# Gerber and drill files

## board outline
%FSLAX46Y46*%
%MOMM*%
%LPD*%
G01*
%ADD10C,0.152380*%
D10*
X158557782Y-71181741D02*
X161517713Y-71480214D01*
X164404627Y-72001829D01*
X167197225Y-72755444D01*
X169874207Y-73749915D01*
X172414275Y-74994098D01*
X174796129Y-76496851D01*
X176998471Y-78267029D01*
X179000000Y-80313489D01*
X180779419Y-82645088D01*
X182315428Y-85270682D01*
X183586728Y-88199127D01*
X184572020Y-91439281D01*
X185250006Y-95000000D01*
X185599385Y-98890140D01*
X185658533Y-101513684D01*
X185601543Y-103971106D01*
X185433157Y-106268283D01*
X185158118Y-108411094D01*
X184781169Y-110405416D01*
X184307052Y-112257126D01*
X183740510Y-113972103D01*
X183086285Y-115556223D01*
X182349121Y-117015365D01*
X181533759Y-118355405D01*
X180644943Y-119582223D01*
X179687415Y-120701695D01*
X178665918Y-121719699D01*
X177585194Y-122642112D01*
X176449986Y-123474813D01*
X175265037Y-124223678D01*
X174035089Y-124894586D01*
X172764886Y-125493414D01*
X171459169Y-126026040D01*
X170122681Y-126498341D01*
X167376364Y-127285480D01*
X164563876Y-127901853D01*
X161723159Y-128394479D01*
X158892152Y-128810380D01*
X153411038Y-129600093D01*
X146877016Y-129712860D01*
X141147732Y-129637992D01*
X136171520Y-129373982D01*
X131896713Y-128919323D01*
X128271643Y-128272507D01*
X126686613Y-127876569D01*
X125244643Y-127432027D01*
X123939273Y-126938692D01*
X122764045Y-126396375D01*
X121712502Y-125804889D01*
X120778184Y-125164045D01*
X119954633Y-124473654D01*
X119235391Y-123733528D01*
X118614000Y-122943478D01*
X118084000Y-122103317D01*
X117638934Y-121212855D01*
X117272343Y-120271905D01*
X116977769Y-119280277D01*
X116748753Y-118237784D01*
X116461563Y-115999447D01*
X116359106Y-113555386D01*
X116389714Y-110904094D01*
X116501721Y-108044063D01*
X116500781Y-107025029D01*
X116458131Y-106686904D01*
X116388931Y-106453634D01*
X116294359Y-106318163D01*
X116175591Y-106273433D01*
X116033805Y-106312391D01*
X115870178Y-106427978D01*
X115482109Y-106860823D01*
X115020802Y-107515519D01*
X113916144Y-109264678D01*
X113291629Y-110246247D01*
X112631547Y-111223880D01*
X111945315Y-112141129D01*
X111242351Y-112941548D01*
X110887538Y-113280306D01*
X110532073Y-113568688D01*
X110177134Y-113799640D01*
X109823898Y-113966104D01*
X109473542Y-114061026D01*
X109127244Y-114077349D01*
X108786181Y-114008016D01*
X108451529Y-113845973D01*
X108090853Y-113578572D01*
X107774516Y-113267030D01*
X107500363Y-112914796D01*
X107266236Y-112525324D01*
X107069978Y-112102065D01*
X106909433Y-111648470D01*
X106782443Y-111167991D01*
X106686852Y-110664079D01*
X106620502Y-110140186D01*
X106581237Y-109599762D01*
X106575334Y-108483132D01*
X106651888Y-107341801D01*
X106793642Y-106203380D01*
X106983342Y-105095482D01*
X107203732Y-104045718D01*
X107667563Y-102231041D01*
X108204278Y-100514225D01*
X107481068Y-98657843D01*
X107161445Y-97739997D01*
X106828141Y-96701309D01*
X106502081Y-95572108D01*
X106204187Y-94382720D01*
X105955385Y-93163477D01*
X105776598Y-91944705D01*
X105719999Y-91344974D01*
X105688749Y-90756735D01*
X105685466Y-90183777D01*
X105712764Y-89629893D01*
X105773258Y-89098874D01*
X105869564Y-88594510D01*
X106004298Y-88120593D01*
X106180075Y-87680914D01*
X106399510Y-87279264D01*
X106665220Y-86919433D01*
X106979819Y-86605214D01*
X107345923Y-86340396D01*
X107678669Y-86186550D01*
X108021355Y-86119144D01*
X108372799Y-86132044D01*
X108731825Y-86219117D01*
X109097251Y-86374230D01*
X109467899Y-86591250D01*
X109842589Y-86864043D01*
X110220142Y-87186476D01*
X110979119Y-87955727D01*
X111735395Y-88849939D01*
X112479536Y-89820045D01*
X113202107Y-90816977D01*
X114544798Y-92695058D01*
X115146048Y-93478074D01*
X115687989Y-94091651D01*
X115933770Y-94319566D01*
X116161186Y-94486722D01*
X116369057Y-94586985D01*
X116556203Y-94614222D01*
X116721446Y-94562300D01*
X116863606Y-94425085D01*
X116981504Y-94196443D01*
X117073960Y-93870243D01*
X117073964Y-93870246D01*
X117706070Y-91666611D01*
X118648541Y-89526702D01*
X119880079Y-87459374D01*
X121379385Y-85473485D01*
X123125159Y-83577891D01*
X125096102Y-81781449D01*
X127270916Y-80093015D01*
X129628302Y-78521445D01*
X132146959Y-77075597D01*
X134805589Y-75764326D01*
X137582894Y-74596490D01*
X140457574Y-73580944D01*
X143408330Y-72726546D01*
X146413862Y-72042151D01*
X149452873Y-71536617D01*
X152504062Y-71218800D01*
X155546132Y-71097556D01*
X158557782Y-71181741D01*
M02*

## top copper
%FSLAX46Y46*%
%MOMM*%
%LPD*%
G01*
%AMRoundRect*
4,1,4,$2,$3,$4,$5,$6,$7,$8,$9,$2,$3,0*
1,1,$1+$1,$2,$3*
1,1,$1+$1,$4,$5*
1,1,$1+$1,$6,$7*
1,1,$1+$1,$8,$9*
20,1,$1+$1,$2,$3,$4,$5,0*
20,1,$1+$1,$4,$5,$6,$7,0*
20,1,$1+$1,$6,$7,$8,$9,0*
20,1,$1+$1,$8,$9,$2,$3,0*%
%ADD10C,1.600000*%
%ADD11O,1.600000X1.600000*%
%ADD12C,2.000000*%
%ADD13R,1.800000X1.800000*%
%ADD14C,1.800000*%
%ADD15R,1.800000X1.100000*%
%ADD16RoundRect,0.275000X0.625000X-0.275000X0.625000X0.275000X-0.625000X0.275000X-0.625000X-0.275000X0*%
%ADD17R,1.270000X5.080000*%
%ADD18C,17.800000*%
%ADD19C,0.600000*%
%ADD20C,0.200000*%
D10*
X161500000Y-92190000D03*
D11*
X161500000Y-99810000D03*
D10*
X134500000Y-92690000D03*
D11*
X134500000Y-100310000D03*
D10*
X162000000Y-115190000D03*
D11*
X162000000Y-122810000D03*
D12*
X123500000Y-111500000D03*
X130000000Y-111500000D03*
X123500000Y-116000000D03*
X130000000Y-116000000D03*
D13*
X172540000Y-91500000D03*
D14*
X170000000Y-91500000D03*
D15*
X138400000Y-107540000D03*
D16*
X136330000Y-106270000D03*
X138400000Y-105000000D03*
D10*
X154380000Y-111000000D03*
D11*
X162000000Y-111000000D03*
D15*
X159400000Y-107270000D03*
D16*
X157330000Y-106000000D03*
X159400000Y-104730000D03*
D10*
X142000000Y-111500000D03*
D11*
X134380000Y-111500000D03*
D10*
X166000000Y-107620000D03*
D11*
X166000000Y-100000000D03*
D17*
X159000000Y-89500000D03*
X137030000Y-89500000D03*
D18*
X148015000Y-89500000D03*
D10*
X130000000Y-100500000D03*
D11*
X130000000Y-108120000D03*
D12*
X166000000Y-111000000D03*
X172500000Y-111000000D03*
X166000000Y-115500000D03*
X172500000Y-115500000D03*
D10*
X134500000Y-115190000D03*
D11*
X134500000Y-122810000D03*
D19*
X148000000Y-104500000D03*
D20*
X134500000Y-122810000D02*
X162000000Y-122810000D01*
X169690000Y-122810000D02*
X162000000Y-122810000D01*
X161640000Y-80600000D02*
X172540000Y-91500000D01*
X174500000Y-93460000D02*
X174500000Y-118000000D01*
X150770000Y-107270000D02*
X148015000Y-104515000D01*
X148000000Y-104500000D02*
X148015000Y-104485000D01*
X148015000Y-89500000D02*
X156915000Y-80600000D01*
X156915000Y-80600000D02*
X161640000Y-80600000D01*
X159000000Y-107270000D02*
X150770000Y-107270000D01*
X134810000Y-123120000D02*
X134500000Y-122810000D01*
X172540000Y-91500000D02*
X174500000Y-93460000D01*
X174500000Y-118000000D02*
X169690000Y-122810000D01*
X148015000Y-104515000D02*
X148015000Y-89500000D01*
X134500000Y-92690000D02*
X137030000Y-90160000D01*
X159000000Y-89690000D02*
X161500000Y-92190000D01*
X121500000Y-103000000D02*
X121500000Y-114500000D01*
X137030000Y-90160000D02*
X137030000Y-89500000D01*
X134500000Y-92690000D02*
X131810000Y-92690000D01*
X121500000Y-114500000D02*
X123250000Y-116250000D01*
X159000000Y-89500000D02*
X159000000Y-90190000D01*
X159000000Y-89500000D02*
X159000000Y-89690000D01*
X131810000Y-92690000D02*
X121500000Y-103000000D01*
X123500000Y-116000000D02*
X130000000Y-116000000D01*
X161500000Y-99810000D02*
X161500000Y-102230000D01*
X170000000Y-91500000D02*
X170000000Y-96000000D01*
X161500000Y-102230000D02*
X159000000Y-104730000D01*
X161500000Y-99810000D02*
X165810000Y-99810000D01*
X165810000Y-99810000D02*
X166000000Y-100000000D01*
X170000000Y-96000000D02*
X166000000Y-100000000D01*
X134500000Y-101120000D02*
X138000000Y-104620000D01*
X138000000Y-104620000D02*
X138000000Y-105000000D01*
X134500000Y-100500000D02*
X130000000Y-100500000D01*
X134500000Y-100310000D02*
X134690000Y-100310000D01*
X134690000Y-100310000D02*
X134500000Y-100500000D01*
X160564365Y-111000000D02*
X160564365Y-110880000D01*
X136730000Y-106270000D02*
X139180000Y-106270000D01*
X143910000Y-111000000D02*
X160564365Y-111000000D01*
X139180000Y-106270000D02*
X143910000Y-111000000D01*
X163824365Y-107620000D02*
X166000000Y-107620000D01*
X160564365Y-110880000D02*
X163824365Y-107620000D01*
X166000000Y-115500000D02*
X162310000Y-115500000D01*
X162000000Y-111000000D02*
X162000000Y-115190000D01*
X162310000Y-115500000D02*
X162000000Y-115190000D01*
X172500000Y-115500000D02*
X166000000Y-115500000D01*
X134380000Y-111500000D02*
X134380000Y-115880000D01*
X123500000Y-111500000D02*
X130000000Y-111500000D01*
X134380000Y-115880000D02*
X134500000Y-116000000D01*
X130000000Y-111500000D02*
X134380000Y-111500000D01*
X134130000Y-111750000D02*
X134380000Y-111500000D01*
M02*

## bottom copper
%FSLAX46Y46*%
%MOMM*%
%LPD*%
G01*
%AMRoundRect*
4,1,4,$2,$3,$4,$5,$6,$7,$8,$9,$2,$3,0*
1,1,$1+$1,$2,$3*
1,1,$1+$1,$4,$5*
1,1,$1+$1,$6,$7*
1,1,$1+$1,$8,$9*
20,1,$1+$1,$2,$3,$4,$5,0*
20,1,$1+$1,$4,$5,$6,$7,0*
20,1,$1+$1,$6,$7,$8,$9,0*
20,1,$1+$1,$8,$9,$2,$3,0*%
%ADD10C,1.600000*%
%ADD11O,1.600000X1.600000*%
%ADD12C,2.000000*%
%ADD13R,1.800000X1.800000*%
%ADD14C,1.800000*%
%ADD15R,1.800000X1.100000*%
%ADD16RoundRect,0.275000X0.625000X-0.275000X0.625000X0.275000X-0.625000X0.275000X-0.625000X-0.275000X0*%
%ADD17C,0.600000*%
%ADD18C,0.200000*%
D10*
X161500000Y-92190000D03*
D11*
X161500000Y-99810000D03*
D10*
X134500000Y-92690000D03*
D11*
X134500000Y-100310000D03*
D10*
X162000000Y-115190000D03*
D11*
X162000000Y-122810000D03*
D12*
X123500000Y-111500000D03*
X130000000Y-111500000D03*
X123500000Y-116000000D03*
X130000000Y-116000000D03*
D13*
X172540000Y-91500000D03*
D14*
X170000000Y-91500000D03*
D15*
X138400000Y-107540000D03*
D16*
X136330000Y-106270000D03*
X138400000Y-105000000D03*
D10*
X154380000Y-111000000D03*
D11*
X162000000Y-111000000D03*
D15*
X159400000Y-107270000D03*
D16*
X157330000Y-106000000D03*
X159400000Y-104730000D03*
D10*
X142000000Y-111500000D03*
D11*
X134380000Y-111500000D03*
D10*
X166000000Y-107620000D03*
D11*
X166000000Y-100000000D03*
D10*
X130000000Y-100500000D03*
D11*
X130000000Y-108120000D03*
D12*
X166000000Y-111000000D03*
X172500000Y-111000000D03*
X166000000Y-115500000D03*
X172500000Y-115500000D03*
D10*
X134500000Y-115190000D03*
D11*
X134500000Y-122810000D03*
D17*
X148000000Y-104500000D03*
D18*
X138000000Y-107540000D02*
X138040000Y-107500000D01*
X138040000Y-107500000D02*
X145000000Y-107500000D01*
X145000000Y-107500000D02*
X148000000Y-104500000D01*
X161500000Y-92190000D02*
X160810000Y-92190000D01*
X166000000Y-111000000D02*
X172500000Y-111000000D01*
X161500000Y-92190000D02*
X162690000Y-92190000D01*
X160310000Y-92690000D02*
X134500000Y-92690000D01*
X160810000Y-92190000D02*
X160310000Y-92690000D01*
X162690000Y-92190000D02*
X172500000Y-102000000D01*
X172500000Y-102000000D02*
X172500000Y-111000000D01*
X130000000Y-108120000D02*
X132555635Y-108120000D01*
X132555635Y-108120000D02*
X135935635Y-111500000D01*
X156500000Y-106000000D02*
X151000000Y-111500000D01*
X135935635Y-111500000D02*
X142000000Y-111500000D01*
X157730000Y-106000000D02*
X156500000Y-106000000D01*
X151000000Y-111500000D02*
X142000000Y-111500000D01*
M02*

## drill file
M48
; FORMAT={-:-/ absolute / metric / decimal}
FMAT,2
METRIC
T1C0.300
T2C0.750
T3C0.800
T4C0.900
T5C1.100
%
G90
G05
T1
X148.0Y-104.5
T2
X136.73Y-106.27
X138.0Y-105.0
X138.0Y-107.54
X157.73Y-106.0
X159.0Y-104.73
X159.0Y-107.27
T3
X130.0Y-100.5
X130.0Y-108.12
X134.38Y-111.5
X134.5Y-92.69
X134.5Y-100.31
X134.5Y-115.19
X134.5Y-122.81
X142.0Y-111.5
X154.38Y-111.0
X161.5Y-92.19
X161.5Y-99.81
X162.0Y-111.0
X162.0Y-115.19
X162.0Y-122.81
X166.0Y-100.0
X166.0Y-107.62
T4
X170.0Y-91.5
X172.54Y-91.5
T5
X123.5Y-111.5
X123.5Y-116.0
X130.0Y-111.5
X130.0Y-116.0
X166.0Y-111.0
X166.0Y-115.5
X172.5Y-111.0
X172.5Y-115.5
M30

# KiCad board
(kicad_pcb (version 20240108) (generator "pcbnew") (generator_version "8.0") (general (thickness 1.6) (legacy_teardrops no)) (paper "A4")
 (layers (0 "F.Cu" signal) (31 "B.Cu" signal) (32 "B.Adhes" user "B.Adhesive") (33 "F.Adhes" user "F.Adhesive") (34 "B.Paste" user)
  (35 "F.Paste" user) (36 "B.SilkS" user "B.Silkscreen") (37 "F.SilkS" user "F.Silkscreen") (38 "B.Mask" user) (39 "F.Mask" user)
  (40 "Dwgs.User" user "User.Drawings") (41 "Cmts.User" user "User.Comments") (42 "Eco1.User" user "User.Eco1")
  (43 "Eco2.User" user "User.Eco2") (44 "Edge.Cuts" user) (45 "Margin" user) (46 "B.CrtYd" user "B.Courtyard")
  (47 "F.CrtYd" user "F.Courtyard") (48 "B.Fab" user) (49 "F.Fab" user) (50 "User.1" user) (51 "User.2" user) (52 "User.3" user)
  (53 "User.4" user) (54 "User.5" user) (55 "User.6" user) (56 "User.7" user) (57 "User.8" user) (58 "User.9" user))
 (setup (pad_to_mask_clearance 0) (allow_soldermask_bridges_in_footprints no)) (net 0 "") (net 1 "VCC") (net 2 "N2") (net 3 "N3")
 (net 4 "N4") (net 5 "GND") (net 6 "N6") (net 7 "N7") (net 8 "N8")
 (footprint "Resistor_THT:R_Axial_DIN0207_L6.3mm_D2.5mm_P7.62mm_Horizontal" (layer "F.Cu") (at 161.5 92.19 -90)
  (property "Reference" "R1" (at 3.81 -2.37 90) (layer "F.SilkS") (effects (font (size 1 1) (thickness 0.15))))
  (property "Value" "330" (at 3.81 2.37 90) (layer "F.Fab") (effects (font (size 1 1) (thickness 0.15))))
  (pad "1" thru_hole circle (at 0 0 270) (size 1.6 1.6) (drill 0.8) (layers "*.Cu" "*.Mask") (remove_unused_layers no) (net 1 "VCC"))
  (pad "2" thru_hole oval (at 7.62 0 270) (size 1.6 1.6) (drill 0.8) (layers "*.Cu" "*.Mask") (remove_unused_layers no) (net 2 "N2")))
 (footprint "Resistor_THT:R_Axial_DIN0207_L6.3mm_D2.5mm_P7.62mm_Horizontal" (layer "F.Cu") (at 134.5 92.69 -90)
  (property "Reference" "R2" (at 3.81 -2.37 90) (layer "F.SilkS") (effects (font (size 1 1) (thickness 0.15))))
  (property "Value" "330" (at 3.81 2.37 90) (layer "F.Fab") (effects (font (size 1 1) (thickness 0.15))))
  (pad "1" thru_hole circle (at 0 0 270) (size 1.6 1.6) (drill 0.8) (layers "*.Cu" "*.Mask") (remove_unused_layers no) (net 1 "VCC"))
  (pad "2" thru_hole oval (at 7.62 0 270) (size 1.6 1.6) (drill 0.8) (layers "*.Cu" "*.Mask") (remove_unused_layers no) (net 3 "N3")))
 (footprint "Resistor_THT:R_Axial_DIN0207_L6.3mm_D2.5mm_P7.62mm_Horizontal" (layer "F.Cu") (at 162 115.19 -90)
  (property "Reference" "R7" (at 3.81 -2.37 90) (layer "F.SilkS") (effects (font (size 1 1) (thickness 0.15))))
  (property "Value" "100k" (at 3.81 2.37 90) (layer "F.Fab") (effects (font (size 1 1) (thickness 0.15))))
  (pad "1" thru_hole circle (at 0 0 270) (size 1.6 1.6) (drill 0.8) (layers "*.Cu" "*.Mask") (remove_unused_layers no) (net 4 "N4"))
  (pad "2" thru_hole oval (at 7.62 0 270) (size 1.6 1.6) (drill 0.8) (layers "*.Cu" "*.Mask") (remove_unused_layers no) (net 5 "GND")))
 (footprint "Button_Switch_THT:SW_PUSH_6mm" (layer "F.Cu") (at 123.5 111.5)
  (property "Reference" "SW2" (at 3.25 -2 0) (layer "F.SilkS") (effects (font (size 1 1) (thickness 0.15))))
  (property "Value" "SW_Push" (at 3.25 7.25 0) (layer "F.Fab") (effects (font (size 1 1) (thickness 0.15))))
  (pad "1" thru_hole circle (at 0 0 90) (size 2 2) (drill 1.1) (layers "*.Cu" "*.Mask") (remove_unused_layers no) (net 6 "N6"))
  (pad "1" thru_hole circle (at 6.5 0 90) (size 2 2) (drill 1.1) (layers "*.Cu" "*.Mask") (remove_unused_layers no) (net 6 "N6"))
  (pad "2" thru_hole circle (at 0 4.5 90) (size 2 2) (drill 1.1) (layers "*.Cu" "*.Mask") (remove_unused_layers no) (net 1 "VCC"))
  (pad "2" thru_hole circle (at 6.5 4.5 90) (size 2 2) (drill 1.1) (layers "*.Cu" "*.Mask") (remove_unused_layers no) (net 1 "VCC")))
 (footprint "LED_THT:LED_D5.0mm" (layer "F.Cu") (at 172.54 91.5 180)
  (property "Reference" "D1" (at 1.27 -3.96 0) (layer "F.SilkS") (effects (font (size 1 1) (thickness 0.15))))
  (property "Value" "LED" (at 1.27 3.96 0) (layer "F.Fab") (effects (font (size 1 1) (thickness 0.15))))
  (pad "1" thru_hole rect (at 0 0 180) (size 1.8 1.8) (drill 0.9) (layers "*.Cu" "*.Mask") (remove_unused_layers no) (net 5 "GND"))
  (pad "2" thru_hole circle (at 2.54 0 180) (size 1.8 1.8) (drill 0.9) (layers "*.Cu" "*.Mask") (remove_unused_layers no) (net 2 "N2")))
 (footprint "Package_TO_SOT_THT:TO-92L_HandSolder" (layer "F.Cu") (at 138 107.54 90)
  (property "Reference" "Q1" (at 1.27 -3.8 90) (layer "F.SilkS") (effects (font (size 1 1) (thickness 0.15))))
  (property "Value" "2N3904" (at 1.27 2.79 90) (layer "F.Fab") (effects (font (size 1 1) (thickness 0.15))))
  (pad "1" thru_hole rect (at 0 0 90) (size 1.1 1.8) (drill 0.75 (offset 0 0.4)) (layers "*.Cu" "*.Mask") (remove_unused_layers no)
   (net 5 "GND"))
  (pad "2" thru_hole roundrect (at 1.27 -1.27 90) (size 1.1 1.8) (drill 0.75 (offset 0 -0.4)) (layers "*.Cu" "*.Mask")
   (remove_unused_layers no) (roundrect_rratio 0.25) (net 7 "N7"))
  (pad "3" thru_hole roundrect (at 2.54 0 90) (size 1.1 1.8) (drill 0.75 (offset 0 0.4)) (layers "*.Cu" "*.Mask") (remove_unused_layers no)
   (roundrect_rratio 0.25) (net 3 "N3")))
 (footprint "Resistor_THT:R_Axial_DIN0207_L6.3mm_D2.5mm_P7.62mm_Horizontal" (layer "F.Cu") (at 154.38 111)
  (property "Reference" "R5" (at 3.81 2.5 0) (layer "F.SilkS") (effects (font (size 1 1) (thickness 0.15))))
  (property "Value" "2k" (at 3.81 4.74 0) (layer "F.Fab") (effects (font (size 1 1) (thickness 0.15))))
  (pad "1" thru_hole circle (at 0 0) (size 1.6 1.6) (drill 0.8) (layers "*.Cu" "*.Mask") (remove_unused_layers no) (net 7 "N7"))
  (pad "2" thru_hole oval (at 7.62 0) (size 1.6 1.6) (drill 0.8) (layers "*.Cu" "*.Mask") (remove_unused_layers no) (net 4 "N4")))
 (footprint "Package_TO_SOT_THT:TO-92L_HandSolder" (layer "F.Cu") (at 159 107.27 90)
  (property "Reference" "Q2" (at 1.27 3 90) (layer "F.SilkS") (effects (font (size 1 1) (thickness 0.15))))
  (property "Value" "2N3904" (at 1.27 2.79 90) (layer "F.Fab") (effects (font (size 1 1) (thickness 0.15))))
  (pad "1" thru_hole rect (at 0 0 90) (size 1.1 1.8) (drill 0.75 (offset 0 0.4)) (layers "*.Cu" "*.Mask") (remove_unused_layers no)
   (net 5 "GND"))
  (pad "2" thru_hole roundrect (at 1.27 -1.27 90) (size 1.1 1.8) (drill 0.75 (offset 0 -0.4)) (layers "*.Cu" "*.Mask")
   (remove_unused_layers no) (roundrect_rratio 0.25) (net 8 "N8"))
  (pad "3" thru_hole roundrect (at 2.54 0 90) (size 1.1 1.8) (drill 0.75 (offset 0 0.4)) (layers "*.Cu" "*.Mask") (remove_unused_layers no)
   (roundrect_rratio 0.25) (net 2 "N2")))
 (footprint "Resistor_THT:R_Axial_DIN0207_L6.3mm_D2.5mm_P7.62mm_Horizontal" (layer "F.Cu") (at 142 111.5 180)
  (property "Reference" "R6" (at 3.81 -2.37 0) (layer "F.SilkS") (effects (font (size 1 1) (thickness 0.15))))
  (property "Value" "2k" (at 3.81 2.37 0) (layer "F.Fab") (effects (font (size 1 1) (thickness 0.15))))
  (pad "1" thru_hole circle (at 0 0 180) (size 1.6 1.6) (drill 0.8) (layers "*.Cu" "*.Mask") (remove_unused_layers no) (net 8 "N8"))
  (pad "2" thru_hole oval (at 7.62 0 180) (size 1.6 1.6) (drill 0.8) (layers "*.Cu" "*.Mask") (remove_unused_layers no) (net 6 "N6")))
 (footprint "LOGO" (layer "F.Cu") (at 170 81.5)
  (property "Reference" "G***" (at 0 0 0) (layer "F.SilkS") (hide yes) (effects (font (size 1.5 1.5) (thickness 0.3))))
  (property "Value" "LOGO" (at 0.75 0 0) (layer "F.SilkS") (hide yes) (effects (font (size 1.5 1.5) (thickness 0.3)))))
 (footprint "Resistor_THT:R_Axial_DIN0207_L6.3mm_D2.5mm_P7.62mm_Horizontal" (layer "F.Cu") (at 166 107.62 90)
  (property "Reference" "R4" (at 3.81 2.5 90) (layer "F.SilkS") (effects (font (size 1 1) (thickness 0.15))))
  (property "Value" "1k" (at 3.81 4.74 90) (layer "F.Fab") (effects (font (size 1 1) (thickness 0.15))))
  (pad "1" thru_hole circle (at 0 0 90) (size 1.6 1.6) (drill 0.8) (layers "*.Cu" "*.Mask") (remove_unused_layers no) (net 7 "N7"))
  (pad "2" thru_hole oval (at 7.62 0 90) (size 1.6 1.6) (drill 0.8) (layers "*.Cu" "*.Mask") (remove_unused_layers no) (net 2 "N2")))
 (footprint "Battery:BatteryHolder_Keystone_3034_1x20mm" (layer "F.Cu") (at 148.015 89.5 180)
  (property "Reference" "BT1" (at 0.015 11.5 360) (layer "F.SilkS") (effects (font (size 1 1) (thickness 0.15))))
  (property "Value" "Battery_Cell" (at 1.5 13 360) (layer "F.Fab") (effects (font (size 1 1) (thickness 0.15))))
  (pad "1" smd rect (at -10.985 0 180) (size 1.27 5.08) (layers "F.Cu" "F.Paste" "F.Mask") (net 1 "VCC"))
  (pad "1" smd rect (at 10.985 0 180) (size 1.27 5.08) (layers "F.Cu" "F.Paste" "F.Mask") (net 1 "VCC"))
  (pad "2" smd circle (at 0 0 180) (size 17.8 17.8) (layers "F.Cu" "F.Mask") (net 5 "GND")))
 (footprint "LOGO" (layer "F.Cu") (at 126.5 91.5)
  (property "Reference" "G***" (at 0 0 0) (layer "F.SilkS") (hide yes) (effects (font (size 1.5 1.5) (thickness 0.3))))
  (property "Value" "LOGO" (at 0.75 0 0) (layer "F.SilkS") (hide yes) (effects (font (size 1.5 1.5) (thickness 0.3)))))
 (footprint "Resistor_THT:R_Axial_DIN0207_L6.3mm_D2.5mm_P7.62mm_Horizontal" (layer "F.Cu") (at 130 100.5 -90)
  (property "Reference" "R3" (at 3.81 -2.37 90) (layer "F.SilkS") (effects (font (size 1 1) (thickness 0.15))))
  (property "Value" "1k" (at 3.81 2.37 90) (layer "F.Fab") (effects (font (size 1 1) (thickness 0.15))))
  (pad "1" thru_hole circle (at 0 0 270) (size 1.6 1.6) (drill 0.8) (layers "*.Cu" "*.Mask") (remove_unused_layers no) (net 3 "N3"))
  (pad "2" thru_hole oval (at 7.62 0 270) (size 1.6 1.6) (drill 0.8) (layers "*.Cu" "*.Mask") (remove_unused_layers no) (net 8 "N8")))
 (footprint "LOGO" (layer "F.Cu") (at 128.5 122.5)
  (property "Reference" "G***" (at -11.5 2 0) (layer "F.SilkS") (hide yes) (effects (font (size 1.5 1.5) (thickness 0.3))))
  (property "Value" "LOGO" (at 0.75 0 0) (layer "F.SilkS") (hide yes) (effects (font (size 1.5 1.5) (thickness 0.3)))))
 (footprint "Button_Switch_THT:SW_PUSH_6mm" (layer "F.Cu") (at 166 111)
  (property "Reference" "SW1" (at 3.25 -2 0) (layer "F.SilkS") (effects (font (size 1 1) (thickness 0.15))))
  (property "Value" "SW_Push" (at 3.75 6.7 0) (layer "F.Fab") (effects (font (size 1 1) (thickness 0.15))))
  (pad "1" thru_hole circle (at 0 0 90) (size 2 2) (drill 1.1) (layers "*.Cu" "*.Mask") (remove_unused_layers no) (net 1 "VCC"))
  (pad "1" thru_hole circle (at 6.5 0 90) (size 2 2) (drill 1.1) (layers "*.Cu" "*.Mask") (remove_unused_layers no) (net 1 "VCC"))
  (pad "2" thru_hole circle (at 0 4.5 90) (size 2 2) (drill 1.1) (layers "*.Cu" "*.Mask") (remove_unused_layers no) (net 4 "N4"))
  (pad "2" thru_hole circle (at 6.5 4.5 90) (size 2 2) (drill 1.1) (layers "*.Cu" "*.Mask") (remove_unused_layers no) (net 4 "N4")))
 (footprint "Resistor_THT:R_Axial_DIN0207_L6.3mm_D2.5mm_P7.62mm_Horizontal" (layer "F.Cu") (at 134.5 115.19 -90)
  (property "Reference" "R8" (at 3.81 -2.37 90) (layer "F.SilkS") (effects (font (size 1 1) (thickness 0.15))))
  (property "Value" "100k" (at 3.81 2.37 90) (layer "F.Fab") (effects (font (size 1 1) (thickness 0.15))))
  (pad "1" thru_hole circle (at 0 0 270) (size 1.6 1.6) (drill 0.8) (layers "*.Cu" "*.Mask") (remove_unused_layers no) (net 6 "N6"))
  (pad "2" thru_hole oval (at 7.62 0 270) (size 1.6 1.6) (drill 0.8) (layers "*.Cu" "*.Mask") (remove_unused_layers no) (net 5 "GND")))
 (gr_poly
  (pts (xy 158.557782 71.181741) (xy 161.517713 71.480214) (xy 164.404627 72.001829) (xy 167.197225 72.755444) (xy 169.874207 73.749915)
   (xy 172.414275 74.994098) (xy 174.796129 76.496851) (xy 176.998471 78.267029) (xy 179 80.313489) (xy 180.779419 82.645088)
   (xy 182.315428 85.270682) (xy 183.586728 88.199127) (xy 184.57202 91.439281) (xy 185.250006 95) (xy 185.599385 98.89014)
   (xy 185.658533 101.513684) (xy 185.601543 103.971106) (xy 185.433157 106.268283) (xy 185.158118 108.411094) (xy 184.781169 110.405416)
   (xy 184.307052 112.257126) (xy 183.74051 113.972103) (xy 183.086285 115.556223) (xy 182.349121 117.015365) (xy 181.533759 118.355405)
   (xy 180.644943 119.582223) (xy 179.687415 120.701695) (xy 178.665918 121.719699) (xy 177.585194 122.642112) (xy 176.449986 123.474813)
   (xy 175.265037 124.223678) (xy 174.035089 124.894586) (xy 172.764886 125.493414) (xy 171.459169 126.02604) (xy 170.122681 126.498341)
   (xy 167.376364 127.28548) (xy 164.563876 127.901853) (xy 161.723159 128.394479) (xy 158.892152 128.81038) (xy 153.411038 129.600093)
   (xy 146.877016 129.71286) (xy 141.147732 129.637992) (xy 136.17152 129.373982) (xy 131.896713 128.919323) (xy 128.271643 128.272507)
   (xy 126.686613 127.876569) (xy 125.244643 127.432027) (xy 123.939273 126.938692) (xy 122.764045 126.396375) (xy 121.712502 125.804889)
   (xy 120.778184 125.164045) (xy 119.954633 124.473654) (xy 119.235391 123.733528) (xy 118.614 122.943478) (xy 118.084 122.103317)
   (xy 117.638934 121.212855) (xy 117.272343 120.271905) (xy 116.977769 119.280277) (xy 116.748753 118.237784) (xy 116.461563 115.999447)
   (xy 116.359106 113.555386) (xy 116.389714 110.904094) (xy 116.501721 108.044063) (xy 116.500781 107.025029) (xy 116.458131 106.686904)
   (xy 116.388931 106.453634) (xy 116.294359 106.318163) (xy 116.175591 106.273433) (xy 116.033805 106.312391) (xy 115.870178 106.427978)
   (xy 115.482109 106.860823) (xy 115.020802 107.515519) (xy 113.916144 109.264678) (xy 113.291629 110.246247) (xy 112.631547 111.22388)
   (xy 111.945315 112.141129) (xy 111.242351 112.941548) (xy 110.887538 113.280306) (xy 110.532073 113.568688) (xy 110.177134 113.79964)
   (xy 109.823898 113.966104) (xy 109.473542 114.061026) (xy 109.127244 114.077349) (xy 108.786181 114.008016) (xy 108.451529 113.845973)
   (xy 108.090853 113.578572) (xy 107.774516 113.26703) (xy 107.500363 112.914796) (xy 107.266236 112.525324) (xy 107.069978 112.102065)
   (xy 106.909433 111.64847) (xy 106.782443 111.167991) (xy 106.686852 110.664079) (xy 106.620502 110.140186) (xy 106.581237 109.599762)
   (xy 106.575334 108.483132) (xy 106.651888 107.341801) (xy 106.793642 106.20338) (xy 106.983342 105.095482) (xy 107.203732 104.045718)
   (xy 107.667563 102.231041) (xy 108.204278 100.514225) (xy 107.481068 98.657843) (xy 107.161445 97.739997) (xy 106.828141 96.701309)
   (xy 106.502081 95.572108) (xy 106.204187 94.38272) (xy 105.955385 93.163477) (xy 105.776598 91.944705) (xy 105.719999 91.344974)
   (xy 105.688749 90.756735) (xy 105.685466 90.183777) (xy 105.712764 89.629893) (xy 105.773258 89.098874) (xy 105.869564 88.59451)
   (xy 106.004298 88.120593) (xy 106.180075 87.680914) (xy 106.39951 87.279264) (xy 106.66522 86.919433) (xy 106.979819 86.605214)
   (xy 107.345923 86.340396) (xy 107.678669 86.18655) (xy 108.021355 86.119144) (xy 108.372799 86.132044) (xy 108.731825 86.219117)
   (xy 109.097251 86.37423) (xy 109.467899 86.59125) (xy 109.842589 86.864043) (xy 110.220142 87.186476) (xy 110.979119 87.955727)
   (xy 111.735395 88.849939) (xy 112.479536 89.820045) (xy 113.202107 90.816977) (xy 114.544798 92.695058) (xy 115.146048 93.478074)
   (xy 115.687989 94.091651) (xy 115.93377 94.319566) (xy 116.161186 94.486722) (xy 116.369057 94.586985) (xy 116.556203 94.614222)
   (xy 116.721446 94.5623) (xy 116.863606 94.425085) (xy 116.981504 94.196443) (xy 117.07396 93.870243) (xy 117.073964 93.870246)
   (xy 117.70607 91.666611) (xy 118.648541 89.526702) (xy 119.880079 87.459374) (xy 121.379385 85.473485) (xy 123.125159 83.577891)
   (xy 125.096102 81.781449) (xy 127.270916 80.093015) (xy 129.628302 78.521445) (xy 132.146959 77.075597) (xy 134.805589 75.764326)
   (xy 137.582894 74.59649) (xy 140.457574 73.580944) (xy 143.40833 72.726546) (xy 146.413862 72.042151) (xy 149.452873 71.536617)
   (xy 152.504062 71.2188) (xy 155.546132 71.097556))
  (stroke (width 0.15238) (type solid) (color 255 0 0 1)) (fill none) (layer "Edge.Cuts"))
 (segment (start 134.5 122.81) (end 162 122.81) (width 0.2) (layer "F.Cu") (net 5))
 (segment (start 169.69 122.81) (end 162 122.81) (width 0.2) (layer "F.Cu") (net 5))
 (segment (start 161.64 80.6) (end 172.54 91.5) (width 0.2) (layer "F.Cu") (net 5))
 (segment (start 174.5 93.46) (end 174.5 118) (width 0.2) (layer "F.Cu") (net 5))
 (segment (start 150.77 107.27) (end 148.015 104.515) (width 0.2) (layer "F.Cu") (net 5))
 (segment (start 148 104.5) (end 148.015 104.485) (width 0.2) (layer "F.Cu") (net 5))
 (segment (start 148.015 89.5) (end 156.915 80.6) (width 0.2) (layer "F.Cu") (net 5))
 (segment (start 156.915 80.6) (end 161.64 80.6) (width 0.2) (layer "F.Cu") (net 5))
 (segment (start 159 107.27) (end 150.77 107.27) (width 0.2) (layer "F.Cu") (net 5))
 (segment (start 134.81 123.12) (end 134.5 122.81) (width 0.2) (layer "F.Cu") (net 5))
 (segment (start 172.54 91.5) (end 174.5 93.46) (width 0.2) (layer "F.Cu") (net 5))
 (segment (start 174.5 118) (end 169.69 122.81) (width 0.2) (layer "F.Cu") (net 5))
 (segment (start 148.015 104.515) (end 148.015 89.5) (width 0.2) (layer "F.Cu") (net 5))
 (via (at 148 104.5) (size 0.6) (drill 0.3) (layers "F.Cu" "B.Cu") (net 5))
 (segment (start 138 107.54) (end 138.04 107.5) (width 0.2) (layer "B.Cu") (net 5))
 (segment (start 138.04 107.5) (end 145 107.5) (width 0.2) (layer "B.Cu") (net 5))
 (segment (start 145 107.5) (end 148 104.5) (width 0.2) (layer "B.Cu") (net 5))
 (segment (start 134.5 92.69) (end 137.03 90.16) (width 0.2) (layer "F.Cu") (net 1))
 (segment (start 159 89.69) (end 161.5 92.19) (width 0.2) (layer "F.Cu") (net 1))
 (segment (start 121.5 103) (end 121.5 114.5) (width 0.2) (layer "F.Cu") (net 1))
 (segment (start 137.03 90.16) (end 137.03 89.5) (width 0.2) (layer "F.Cu") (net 1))
 (segment (start 134.5 92.69) (end 131.81 92.69) (width 0.2) (layer "F.Cu") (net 1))
 (segment (start 121.5 114.5) (end 123.25 116.25) (width 0.2) (layer "F.Cu") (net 1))
 (segment (start 159 89.5) (end 159 90.19) (width 0.2) (layer "F.Cu") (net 1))
 (segment (start 159 89.5) (end 159 89.69) (width 0.2) (layer "F.Cu") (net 1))
 (segment (start 131.81 92.69) (end 121.5 103) (width 0.2) (layer "F.Cu") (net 1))
 (segment (start 123.5 116) (end 130 116) (width 0.2) (layer "F.Cu") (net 1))
 (segment (start 161.5 92.19) (end 160.81 92.19) (width 0.2) (layer "B.Cu") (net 1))
 (segment (start 166 111) (end 172.5 111) (width 0.2) (layer "B.Cu") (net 1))
 (segment (start 161.5 92.19) (end 162.69 92.19) (width 0.2) (layer "B.Cu") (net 1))
 (segment (start 160.31 92.69) (end 134.5 92.69) (width 0.2) (layer "B.Cu") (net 1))
 (segment (start 160.81 92.19) (end 160.31 92.69) (width 0.2) (layer "B.Cu") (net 1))
 (segment (start 162.69 92.19) (end 172.5 102) (width 0.2) (layer "B.Cu") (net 1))
 (segment (start 172.5 102) (end 172.5 111) (width 0.2) (layer "B.Cu") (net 1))
 (segment (start 161.5 99.81) (end 161.5 102.23) (width 0.2) (layer "F.Cu") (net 2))
 (segment (start 170 91.5) (end 170 96) (width 0.2) (layer "F.Cu") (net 2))
 (segment (start 161.5 102.23) (end 159 104.73) (width 0.2) (layer "F.Cu") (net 2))
 (segment (start 161.5 99.81) (end 165.81 99.81) (width 0.2) (layer "F.Cu") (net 2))
 (segment (start 165.81 99.81) (end 166 100) (width 0.2) (layer "F.Cu") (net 2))
 (segment (start 170 96) (end 166 100) (width 0.2) (layer "F.Cu") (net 2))
 (segment (start 134.5 101.12) (end 138 104.62) (width 0.2) (layer "F.Cu") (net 3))
 (segment (start 138 104.62) (end 138 105) (width 0.2) (layer "F.Cu") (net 3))
 (segment (start 134.5 100.5) (end 130 100.5) (width 0.2) (layer "F.Cu") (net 3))
 (segment (start 134.5 100.31) (end 134.69 100.31) (width 0.2) (layer "F.Cu") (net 3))
 (segment (start 134.69 100.31) (end 134.5 100.5) (width 0.2) (layer "F.Cu") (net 3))
 (segment (start 160.564365 111) (end 160.564365 110.88) (width 0.2) (layer "F.Cu") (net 7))
 (segment (start 136.73 106.27) (end 139.18 106.27) (width 0.2) (layer "F.Cu") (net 7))
 (segment (start 143.91 111) (end 160.564365 111) (width 0.2) (layer "F.Cu") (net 7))
 (segment (start 139.18 106.27) (end 143.91 111) (width 0.2) (layer "F.Cu") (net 7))
 (segment (start 163.824365 107.62) (end 166 107.62) (width 0.2) (layer "F.Cu") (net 7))
 (segment (start 160.564365 110.88) (end 163.824365 107.62) (width 0.2) (layer "F.Cu") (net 7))
 (segment (start 130 108.12) (end 132.555635 108.12) (width 0.2) (layer "B.Cu") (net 8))
 (segment (start 132.555635 108.12) (end 135.935635 111.5) (width 0.2) (layer "B.Cu") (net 8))
 (segment (start 156.5 106) (end 151 111.5) (width 0.2) (layer "B.Cu") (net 8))
 (segment (start 135.935635 111.5) (end 142 111.5) (width 0.2) (layer "B.Cu") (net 8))
 (segment (start 157.73 106) (end 156.5 106) (width 0.2) (layer "B.Cu") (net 8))
 (segment (start 151 111.5) (end 142 111.5) (width 0.2) (layer "B.Cu") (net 8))
 (segment (start 166 115.5) (end 162.31 115.5) (width 0.2) (layer "F.Cu") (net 4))
 (segment (start 162 111) (end 162 115.19) (width 0.2) (layer "F.Cu") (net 4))
 (segment (start 162.31 115.5) (end 162 115.19) (width 0.2) (layer "F.Cu") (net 4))
 (segment (start 172.5 115.5) (end 166 115.5) (width 0.2) (layer "F.Cu") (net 4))
 (segment (start 134.38 111.5) (end 134.38 115.88) (width 0.2) (layer "F.Cu") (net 6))
 (segment (start 123.5 111.5) (end 130 111.5) (width 0.2) (layer "F.Cu") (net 6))
 (segment (start 134.38 115.88) (end 134.5 116) (width 0.2) (layer "F.Cu") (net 6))
 (segment (start 130 111.5) (end 134.38 111.5) (width 0.2) (layer "F.Cu") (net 6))
 (segment (start 134.13 111.75) (end 134.38 111.5) (width 0.2) (layer "F.Cu") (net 6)))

